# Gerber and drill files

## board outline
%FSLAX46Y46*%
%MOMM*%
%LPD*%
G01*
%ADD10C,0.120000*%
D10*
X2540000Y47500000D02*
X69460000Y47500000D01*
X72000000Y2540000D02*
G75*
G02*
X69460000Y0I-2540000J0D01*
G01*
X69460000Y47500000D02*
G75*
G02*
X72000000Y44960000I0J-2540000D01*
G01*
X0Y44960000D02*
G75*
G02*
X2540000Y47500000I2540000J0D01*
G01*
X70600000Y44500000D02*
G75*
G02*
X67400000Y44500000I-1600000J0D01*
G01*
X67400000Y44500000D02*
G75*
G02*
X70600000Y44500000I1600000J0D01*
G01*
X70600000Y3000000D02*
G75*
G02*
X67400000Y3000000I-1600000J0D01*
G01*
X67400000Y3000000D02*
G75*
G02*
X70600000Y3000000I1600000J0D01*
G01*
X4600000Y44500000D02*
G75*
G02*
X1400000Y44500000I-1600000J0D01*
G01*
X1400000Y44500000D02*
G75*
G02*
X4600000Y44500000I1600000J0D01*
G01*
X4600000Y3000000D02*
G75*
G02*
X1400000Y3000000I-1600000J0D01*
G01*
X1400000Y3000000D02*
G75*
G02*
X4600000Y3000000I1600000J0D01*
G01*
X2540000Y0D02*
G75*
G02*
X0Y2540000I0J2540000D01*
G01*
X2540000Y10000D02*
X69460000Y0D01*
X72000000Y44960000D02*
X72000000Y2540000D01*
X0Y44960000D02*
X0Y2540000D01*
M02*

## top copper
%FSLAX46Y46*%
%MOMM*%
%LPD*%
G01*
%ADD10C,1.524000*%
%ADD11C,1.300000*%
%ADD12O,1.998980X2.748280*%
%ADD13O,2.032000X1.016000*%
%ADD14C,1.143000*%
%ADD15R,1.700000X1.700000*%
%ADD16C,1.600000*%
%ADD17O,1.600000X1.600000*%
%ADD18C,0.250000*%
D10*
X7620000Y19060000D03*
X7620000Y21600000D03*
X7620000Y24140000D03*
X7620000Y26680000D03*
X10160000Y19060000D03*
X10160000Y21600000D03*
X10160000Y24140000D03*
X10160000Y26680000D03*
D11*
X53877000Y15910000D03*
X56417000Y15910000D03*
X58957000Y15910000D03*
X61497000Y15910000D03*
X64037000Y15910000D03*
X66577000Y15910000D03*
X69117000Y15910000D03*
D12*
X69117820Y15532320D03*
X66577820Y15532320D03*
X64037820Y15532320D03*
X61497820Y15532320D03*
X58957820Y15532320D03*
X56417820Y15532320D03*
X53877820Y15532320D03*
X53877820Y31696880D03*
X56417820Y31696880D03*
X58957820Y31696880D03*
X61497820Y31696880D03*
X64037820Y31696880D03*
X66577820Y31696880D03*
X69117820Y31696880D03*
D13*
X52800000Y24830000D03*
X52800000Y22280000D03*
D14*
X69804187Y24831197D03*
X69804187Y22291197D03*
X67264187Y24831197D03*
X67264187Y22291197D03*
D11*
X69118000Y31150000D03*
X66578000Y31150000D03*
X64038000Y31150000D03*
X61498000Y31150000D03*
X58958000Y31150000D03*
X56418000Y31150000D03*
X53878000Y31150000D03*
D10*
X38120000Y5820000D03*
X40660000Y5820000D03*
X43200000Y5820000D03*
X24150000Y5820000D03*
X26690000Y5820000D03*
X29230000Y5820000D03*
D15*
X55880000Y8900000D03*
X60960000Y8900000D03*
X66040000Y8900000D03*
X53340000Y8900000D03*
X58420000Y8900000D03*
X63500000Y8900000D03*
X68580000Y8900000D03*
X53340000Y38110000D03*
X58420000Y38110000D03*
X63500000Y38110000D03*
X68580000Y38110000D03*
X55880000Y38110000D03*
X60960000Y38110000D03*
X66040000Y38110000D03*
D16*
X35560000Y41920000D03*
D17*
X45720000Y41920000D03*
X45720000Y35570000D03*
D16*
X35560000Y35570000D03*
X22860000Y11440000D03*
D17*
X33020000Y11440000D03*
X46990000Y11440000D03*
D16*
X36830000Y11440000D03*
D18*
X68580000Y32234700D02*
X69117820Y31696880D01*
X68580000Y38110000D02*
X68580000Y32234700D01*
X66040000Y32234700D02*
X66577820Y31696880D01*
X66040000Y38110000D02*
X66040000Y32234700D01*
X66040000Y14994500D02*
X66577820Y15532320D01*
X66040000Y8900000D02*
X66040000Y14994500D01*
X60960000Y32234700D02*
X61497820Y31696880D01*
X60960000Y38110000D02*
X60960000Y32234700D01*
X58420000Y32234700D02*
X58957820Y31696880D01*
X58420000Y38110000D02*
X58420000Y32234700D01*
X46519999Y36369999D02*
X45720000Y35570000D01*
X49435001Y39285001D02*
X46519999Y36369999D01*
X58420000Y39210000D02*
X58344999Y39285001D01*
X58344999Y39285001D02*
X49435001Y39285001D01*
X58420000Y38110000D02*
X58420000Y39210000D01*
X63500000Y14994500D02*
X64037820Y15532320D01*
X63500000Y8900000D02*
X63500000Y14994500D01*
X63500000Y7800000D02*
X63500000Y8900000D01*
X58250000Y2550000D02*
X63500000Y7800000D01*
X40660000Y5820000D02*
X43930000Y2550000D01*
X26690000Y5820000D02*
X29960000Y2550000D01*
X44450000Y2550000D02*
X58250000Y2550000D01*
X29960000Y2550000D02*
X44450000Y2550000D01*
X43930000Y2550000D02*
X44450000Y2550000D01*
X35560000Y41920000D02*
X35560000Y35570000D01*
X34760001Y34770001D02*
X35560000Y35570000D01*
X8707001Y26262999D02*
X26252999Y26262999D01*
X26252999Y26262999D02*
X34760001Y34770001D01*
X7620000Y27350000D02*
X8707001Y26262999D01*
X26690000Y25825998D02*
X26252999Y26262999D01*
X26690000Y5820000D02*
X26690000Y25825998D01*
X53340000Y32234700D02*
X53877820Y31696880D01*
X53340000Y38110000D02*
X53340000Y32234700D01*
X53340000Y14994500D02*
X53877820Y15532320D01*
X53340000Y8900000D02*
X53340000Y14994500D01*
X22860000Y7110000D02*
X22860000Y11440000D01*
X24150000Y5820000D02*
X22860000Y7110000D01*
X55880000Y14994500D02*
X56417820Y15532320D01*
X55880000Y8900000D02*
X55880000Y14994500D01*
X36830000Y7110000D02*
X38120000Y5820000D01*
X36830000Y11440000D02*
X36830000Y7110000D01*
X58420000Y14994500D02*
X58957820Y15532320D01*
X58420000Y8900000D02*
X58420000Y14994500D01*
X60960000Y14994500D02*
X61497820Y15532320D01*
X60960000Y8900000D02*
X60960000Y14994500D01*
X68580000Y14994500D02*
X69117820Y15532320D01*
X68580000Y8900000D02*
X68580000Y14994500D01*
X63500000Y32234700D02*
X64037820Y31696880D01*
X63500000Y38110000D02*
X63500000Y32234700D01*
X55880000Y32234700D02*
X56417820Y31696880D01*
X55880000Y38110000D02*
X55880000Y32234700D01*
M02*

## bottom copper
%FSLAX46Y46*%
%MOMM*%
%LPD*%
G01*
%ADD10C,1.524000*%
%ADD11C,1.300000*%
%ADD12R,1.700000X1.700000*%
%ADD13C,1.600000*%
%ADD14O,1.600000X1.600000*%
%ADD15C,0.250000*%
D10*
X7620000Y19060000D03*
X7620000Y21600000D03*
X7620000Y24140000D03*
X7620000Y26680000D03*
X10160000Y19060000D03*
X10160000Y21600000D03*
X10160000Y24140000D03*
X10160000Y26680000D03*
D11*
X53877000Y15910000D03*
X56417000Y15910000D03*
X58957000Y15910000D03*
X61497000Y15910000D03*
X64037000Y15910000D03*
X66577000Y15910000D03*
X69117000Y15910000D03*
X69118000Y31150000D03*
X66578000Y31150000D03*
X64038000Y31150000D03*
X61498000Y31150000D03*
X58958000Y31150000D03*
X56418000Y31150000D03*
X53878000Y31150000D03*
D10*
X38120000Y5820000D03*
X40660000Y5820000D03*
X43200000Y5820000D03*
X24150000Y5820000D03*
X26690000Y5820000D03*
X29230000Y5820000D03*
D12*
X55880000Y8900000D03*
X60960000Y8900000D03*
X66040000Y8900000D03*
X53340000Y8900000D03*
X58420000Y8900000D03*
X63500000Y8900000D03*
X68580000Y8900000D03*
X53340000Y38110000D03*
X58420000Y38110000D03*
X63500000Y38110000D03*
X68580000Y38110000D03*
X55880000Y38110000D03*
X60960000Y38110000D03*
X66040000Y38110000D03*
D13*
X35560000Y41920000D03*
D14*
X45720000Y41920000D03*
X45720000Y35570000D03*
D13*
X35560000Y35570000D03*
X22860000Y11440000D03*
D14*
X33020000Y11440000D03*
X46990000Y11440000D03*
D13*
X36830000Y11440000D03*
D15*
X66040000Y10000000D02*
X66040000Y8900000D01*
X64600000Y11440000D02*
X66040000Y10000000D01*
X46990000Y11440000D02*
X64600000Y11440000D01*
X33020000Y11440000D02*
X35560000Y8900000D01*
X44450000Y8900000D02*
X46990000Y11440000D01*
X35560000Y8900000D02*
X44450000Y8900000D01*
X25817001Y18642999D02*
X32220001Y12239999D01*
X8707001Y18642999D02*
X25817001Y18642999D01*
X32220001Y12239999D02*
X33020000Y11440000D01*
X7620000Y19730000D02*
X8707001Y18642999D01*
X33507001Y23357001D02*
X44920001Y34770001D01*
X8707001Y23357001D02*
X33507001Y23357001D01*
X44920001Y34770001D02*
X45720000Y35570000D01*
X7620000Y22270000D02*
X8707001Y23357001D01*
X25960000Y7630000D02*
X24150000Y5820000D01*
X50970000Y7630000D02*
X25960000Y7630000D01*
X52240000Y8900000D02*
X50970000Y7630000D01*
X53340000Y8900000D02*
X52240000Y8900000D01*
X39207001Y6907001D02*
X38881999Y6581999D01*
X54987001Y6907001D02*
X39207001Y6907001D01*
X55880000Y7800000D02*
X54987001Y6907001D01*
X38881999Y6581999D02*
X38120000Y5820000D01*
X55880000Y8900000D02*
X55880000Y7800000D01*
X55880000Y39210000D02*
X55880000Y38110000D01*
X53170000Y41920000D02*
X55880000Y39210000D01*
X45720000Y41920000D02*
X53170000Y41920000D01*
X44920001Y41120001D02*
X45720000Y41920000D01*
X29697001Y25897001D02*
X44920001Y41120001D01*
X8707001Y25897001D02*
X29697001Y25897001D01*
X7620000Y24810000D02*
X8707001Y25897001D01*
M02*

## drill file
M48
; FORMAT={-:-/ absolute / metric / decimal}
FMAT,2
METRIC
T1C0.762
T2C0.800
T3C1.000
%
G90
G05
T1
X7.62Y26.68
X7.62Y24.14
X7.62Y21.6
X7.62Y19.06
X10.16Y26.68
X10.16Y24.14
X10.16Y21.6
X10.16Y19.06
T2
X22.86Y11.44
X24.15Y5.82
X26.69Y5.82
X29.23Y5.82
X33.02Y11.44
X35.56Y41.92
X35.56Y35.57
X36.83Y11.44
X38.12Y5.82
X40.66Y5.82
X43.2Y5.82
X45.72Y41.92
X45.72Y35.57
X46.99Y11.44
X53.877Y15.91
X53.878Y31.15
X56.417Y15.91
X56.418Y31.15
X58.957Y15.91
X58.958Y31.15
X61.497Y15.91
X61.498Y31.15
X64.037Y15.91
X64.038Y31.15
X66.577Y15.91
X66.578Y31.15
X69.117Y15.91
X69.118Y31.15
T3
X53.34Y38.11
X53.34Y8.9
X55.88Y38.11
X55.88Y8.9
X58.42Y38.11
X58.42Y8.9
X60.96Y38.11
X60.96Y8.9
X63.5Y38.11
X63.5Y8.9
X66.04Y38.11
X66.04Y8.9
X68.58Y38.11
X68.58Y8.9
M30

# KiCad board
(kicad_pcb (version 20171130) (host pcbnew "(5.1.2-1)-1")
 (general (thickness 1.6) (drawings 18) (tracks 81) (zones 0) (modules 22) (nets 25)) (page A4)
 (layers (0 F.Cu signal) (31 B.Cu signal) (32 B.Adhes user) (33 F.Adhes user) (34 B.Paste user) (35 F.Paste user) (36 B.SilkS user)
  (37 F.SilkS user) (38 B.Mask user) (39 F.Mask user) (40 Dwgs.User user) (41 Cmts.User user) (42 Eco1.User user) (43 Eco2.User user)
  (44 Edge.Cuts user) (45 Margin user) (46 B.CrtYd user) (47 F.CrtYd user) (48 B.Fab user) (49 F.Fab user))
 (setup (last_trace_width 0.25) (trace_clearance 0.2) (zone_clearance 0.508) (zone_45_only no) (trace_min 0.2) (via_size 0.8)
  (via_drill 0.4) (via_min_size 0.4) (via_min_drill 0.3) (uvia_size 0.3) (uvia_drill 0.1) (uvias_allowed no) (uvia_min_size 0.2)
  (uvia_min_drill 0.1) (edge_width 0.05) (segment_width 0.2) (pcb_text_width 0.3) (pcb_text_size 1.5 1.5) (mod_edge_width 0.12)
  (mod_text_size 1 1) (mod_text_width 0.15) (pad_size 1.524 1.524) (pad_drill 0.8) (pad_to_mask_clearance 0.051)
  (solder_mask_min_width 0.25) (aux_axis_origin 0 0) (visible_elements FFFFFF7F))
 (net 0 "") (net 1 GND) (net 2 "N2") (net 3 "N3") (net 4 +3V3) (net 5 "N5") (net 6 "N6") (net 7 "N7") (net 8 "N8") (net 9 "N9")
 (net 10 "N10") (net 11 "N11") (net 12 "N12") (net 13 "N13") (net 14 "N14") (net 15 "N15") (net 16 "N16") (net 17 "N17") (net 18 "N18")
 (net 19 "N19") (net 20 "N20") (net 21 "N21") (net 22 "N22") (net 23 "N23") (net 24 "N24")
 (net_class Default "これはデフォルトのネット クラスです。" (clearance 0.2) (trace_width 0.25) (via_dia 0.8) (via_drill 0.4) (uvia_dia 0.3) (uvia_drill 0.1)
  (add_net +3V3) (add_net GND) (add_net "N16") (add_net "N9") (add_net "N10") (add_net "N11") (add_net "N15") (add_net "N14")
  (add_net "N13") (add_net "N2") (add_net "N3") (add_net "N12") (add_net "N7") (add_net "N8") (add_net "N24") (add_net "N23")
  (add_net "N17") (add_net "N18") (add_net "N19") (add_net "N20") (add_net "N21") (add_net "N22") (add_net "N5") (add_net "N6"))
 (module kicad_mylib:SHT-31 (layer F.Cu) (at 6.35 -17.79)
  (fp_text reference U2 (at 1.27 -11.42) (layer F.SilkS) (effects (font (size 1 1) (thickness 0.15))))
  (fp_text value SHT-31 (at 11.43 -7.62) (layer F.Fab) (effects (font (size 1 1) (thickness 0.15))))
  (pad 1 thru_hole circle (at 1.27 -1.27) (size 1.524 1.524) (drill 0.762) (layers *.Cu *.Mask) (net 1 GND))
  (pad 2 thru_hole circle (at 1.27 -3.81) (size 1.524 1.524) (drill 0.762) (layers *.Cu *.Mask) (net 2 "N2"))
  (pad 3 thru_hole circle (at 1.27 -6.35) (size 1.524 1.524) (drill 0.762) (layers *.Cu *.Mask) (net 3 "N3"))
  (pad 4 thru_hole circle (at 1.27 -8.89) (size 1.524 1.524) (drill 0.762) (layers *.Cu *.Mask) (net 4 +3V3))
  (pad 5 thru_hole circle (at 3.81 -1.27) (size 1.524 1.524) (drill 0.762) (layers *.Cu *.Mask) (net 1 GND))
  (pad 6 thru_hole circle (at 3.81 -3.81) (size 1.524 1.524) (drill 0.762) (layers *.Cu *.Mask) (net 1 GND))
  (pad 7 thru_hole circle (at 3.81 -6.35) (size 1.524 1.524) (drill 0.762) (layers *.Cu *.Mask) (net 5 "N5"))
  (pad 8 thru_hole circle (at 3.81 -8.89) (size 1.524 1.524) (drill 0.762) (layers *.Cu *.Mask) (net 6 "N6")))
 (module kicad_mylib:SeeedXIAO (layer F.Cu) (at 51 -32.53 270)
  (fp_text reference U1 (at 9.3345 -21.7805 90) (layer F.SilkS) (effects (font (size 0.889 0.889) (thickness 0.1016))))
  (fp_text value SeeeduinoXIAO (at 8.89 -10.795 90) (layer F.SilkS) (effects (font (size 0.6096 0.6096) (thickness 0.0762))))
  (pad 8 thru_hole circle (at 16.62 -2.877 270) (size 1.3 1.3) (drill 0.8) (layers *.Cu *.Mask) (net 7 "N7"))
  (pad 9 thru_hole circle (at 16.62 -5.417 270) (size 1.3 1.3) (drill 0.8) (layers *.Cu *.Mask) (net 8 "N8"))
  (pad 10 thru_hole circle (at 16.62 -7.957 270) (size 1.3 1.3) (drill 0.8) (layers *.Cu *.Mask) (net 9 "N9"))
  (pad 11 thru_hole circle (at 16.62 -10.497 270) (size 1.3 1.3) (drill 0.8) (layers *.Cu *.Mask) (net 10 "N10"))
  (pad 12 thru_hole circle (at 16.62 -13.037 270) (size 1.3 1.3) (drill 0.8) (layers *.Cu *.Mask) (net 4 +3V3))
  (pad 13 thru_hole circle (at 16.62 -15.577 270) (size 1.3 1.3) (drill 0.8) (layers *.Cu *.Mask) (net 1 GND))
  (pad 14 thru_hole circle (at 16.62 -18.117 270) (size 1.3 1.3) (drill 0.8) (layers *.Cu *.Mask) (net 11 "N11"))
  (pad 14 smd oval (at 16.99768 -18.11782 270) (size 2.74828 1.99898) (layers F.Cu F.Paste F.Mask) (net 11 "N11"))
  (pad 13 smd oval (at 16.99768 -15.57782 270) (size 2.74828 1.99898) (layers F.Cu F.Paste F.Mask) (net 1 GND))
  (pad 12 smd oval (at 16.99768 -13.03782 270) (size 2.74828 1.99898) (layers F.Cu F.Paste F.Mask) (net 4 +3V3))
  (pad 11 smd oval (at 16.99768 -10.49782 270) (size 2.74828 1.99898) (layers F.Cu F.Paste F.Mask) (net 10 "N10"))
  (pad 10 smd oval (at 16.99768 -7.95782 270) (size 2.74828 1.99898) (layers F.Cu F.Paste F.Mask) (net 9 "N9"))
  (pad 9 smd oval (at 16.99768 -5.41782 270) (size 2.74828 1.99898) (layers F.Cu F.Paste F.Mask) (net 8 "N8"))
  (pad 8 smd oval (at 16.99768 -2.87782 270) (size 2.74828 1.99898) (layers F.Cu F.Paste F.Mask) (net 7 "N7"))
  (pad 7 smd oval (at 0.83312 -2.87782 270) (size 2.74828 1.99898) (layers F.Cu F.Paste F.Mask) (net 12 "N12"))
  (pad 6 smd oval (at 0.83312 -5.41782 270) (size 2.74828 1.99898) (layers F.Cu F.Paste F.Mask) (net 3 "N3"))
  (pad 5 smd oval (at 0.83312 -7.95782 270) (size 2.74828 1.99898) (layers F.Cu F.Paste F.Mask) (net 2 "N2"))
  (pad 4 smd oval (at 0.83312 -10.49782 270) (size 2.74828 1.99898) (layers F.Cu F.Paste F.Mask) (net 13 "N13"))
  (pad 3 smd oval (at 0.83312 -13.03782 270) (size 2.74828 1.99898) (layers F.Cu F.Paste F.Mask) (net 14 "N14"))
  (pad 2 smd oval (at 0.83312 -15.57782 270) (size 2.74828 1.99898) (layers F.Cu F.Paste F.Mask) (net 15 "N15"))
  (pad 1 smd oval (at 0.83312 -18.11782 270) (size 2.74828 1.99898) (layers F.Cu F.Paste F.Mask) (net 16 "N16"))
  (pad 15 smd oval (at 7.7 -1.8) (size 2.032 1.016) (layers F.Cu F.Paste F.Mask) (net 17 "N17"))
  (pad 16 smd oval (at 10.25 -1.8) (size 2.032 1.016) (layers F.Cu F.Paste F.Mask) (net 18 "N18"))
  (pad 17 smd circle (at 7.698803 -18.804187) (size 1.143 1.143) (layers F.Cu F.Paste F.Mask) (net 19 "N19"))
  (pad 18 smd circle (at 10.238803 -18.804187) (size 1.143 1.143) (layers F.Cu F.Paste F.Mask) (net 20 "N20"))
  (pad 19 smd circle (at 7.698803 -16.264187) (size 1.143 1.143) (layers F.Cu F.Paste F.Mask) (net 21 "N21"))
  (pad 20 smd circle (at 10.238803 -16.264187) (size 1.143 1.143) (layers F.Cu F.Paste F.Mask) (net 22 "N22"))
  (pad 1 thru_hole circle (at 1.38 -18.118 270) (size 1.3 1.3) (drill 0.8) (layers *.Cu *.Mask) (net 16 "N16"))
  (pad 2 thru_hole circle (at 1.38 -15.578 270) (size 1.3 1.3) (drill 0.8) (layers *.Cu *.Mask) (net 15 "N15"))
  (pad 3 thru_hole circle (at 1.38 -13.038 270) (size 1.3 1.3) (drill 0.8) (layers *.Cu *.Mask) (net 14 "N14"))
  (pad 4 thru_hole circle (at 1.38 -10.498 270) (size 1.3 1.3) (drill 0.8) (layers *.Cu *.Mask) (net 13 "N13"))
  (pad 5 thru_hole circle (at 1.38 -7.958 270) (size 1.3 1.3) (drill 0.8) (layers *.Cu *.Mask) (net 2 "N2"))
  (pad 6 thru_hole circle (at 1.38 -5.418 270) (size 1.3 1.3) (drill 0.8) (layers *.Cu *.Mask) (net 3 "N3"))
  (pad 7 thru_hole circle (at 1.38 -2.878 270) (size 1.3 1.3) (drill 0.8) (layers *.Cu *.Mask) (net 12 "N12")))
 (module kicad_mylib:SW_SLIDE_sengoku (layer F.Cu) (at 35.56 -3.82)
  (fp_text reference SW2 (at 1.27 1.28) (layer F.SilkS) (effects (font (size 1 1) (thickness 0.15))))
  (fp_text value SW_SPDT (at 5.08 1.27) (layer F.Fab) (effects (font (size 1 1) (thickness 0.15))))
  (pad 1 thru_hole circle (at 2.56 -2) (size 1.524 1.524) (drill 0.8) (layers *.Cu *.Mask) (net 8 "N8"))
  (pad 2 thru_hole circle (at 5.1 -2) (size 1.524 1.524) (drill 0.8) (layers *.Cu *.Mask) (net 4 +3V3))
  (pad 3 thru_hole circle (at 7.64 -2) (size 1.524 1.524) (drill 0.8) (layers *.Cu *.Mask) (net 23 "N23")))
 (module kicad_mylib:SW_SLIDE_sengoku (layer F.Cu) (at 21.59 -3.82)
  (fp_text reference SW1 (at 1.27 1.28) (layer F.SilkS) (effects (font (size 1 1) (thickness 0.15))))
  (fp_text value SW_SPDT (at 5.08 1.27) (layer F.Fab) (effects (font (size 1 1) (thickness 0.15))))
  (pad 1 thru_hole circle (at 2.56 -2) (size 1.524 1.524) (drill 0.8) (layers *.Cu *.Mask) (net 7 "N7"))
  (pad 2 thru_hole circle (at 5.1 -2) (size 1.524 1.524) (drill 0.8) (layers *.Cu *.Mask) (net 4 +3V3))
  (pad 3 thru_hole circle (at 7.64 -2) (size 1.524 1.524) (drill 0.8) (layers *.Cu *.Mask) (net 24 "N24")))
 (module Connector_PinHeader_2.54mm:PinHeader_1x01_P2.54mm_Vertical (layer F.Cu) (at 55.88 -8.9)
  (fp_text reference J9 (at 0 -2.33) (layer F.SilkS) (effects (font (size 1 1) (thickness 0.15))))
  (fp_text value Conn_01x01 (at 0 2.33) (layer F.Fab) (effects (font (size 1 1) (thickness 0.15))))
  (pad 1 thru_hole rect (at 0 0) (size 1.7 1.7) (drill 1) (layers *.Cu *.Mask) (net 8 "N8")))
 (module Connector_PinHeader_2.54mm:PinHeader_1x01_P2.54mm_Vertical (layer F.Cu) (at 60.96 -8.9)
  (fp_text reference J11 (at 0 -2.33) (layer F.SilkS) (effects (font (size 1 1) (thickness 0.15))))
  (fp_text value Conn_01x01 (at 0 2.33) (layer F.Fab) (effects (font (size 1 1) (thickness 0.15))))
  (pad 1 thru_hole rect (at 0 0) (size 1.7 1.7) (drill 1) (layers *.Cu *.Mask) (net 10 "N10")))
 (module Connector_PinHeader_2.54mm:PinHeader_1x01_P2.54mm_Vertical (layer F.Cu) (at 66.04 -8.9)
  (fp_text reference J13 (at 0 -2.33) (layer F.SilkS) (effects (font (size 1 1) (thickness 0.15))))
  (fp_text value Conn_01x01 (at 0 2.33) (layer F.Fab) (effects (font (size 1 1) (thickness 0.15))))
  (pad 1 thru_hole rect (at 0 0) (size 1.7 1.7) (drill 1) (layers *.Cu *.Mask) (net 1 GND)))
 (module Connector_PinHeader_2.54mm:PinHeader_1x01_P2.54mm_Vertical (layer F.Cu) (at 53.34 -8.9)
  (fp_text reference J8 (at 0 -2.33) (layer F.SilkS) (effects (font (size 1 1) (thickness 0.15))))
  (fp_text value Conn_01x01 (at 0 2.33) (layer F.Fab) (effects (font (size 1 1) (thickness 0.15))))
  (pad 1 thru_hole rect (at 0 0) (size 1.7 1.7) (drill 1) (layers *.Cu *.Mask) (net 7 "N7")))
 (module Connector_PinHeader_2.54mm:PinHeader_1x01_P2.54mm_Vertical (layer F.Cu) (at 58.42 -8.9)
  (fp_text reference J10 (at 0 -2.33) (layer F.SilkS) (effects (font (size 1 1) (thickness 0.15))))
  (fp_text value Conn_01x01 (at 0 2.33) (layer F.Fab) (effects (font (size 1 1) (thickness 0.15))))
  (pad 1 thru_hole rect (at 0 0) (size 1.7 1.7) (drill 1) (layers *.Cu *.Mask) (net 9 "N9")))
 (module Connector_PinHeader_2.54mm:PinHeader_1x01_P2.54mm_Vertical (layer F.Cu) (at 63.5 -8.9)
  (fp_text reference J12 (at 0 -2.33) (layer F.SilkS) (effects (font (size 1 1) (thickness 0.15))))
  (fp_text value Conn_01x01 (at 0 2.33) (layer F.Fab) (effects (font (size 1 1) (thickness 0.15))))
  (pad 1 thru_hole rect (at 0 0) (size 1.7 1.7) (drill 1) (layers *.Cu *.Mask) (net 4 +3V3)))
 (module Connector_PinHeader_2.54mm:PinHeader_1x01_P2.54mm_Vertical (layer F.Cu) (at 68.58 -8.9)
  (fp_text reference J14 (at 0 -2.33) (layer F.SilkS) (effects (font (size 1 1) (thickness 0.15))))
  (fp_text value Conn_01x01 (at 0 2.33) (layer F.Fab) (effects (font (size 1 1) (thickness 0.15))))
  (pad 1 thru_hole rect (at 0 0) (size 1.7 1.7) (drill 1) (layers *.Cu *.Mask) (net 11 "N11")))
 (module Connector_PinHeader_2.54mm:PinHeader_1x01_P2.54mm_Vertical (layer F.Cu) (at 53.34 -38.11)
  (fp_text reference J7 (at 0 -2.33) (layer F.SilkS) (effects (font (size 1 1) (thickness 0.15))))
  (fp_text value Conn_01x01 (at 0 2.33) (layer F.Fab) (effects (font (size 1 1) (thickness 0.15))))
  (pad 1 thru_hole rect (at 0 0) (size 1.7 1.7) (drill 1) (layers *.Cu *.Mask) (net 12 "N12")))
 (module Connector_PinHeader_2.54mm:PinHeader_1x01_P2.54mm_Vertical (layer F.Cu) (at 58.42 -38.11)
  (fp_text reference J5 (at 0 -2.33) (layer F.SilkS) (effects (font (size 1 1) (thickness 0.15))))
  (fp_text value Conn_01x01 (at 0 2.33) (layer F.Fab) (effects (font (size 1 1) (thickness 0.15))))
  (pad 1 thru_hole rect (at 0 0) (size 1.7 1.7) (drill 1) (layers *.Cu *.Mask) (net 2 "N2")))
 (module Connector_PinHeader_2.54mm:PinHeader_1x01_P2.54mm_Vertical (layer F.Cu) (at 63.5 -38.11)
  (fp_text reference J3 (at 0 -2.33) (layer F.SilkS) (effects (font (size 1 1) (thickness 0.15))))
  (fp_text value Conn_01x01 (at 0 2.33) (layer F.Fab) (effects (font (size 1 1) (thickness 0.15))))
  (pad 1 thru_hole rect (at 0 0) (size 1.7 1.7) (drill 1) (layers *.Cu *.Mask) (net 14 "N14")))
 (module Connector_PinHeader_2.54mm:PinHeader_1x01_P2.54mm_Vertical (layer F.Cu) (at 68.58 -38.11)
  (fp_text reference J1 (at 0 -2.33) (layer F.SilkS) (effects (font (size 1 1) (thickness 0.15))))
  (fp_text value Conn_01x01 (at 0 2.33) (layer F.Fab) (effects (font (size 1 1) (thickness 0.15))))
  (pad 1 thru_hole rect (at 0 0) (size 1.7 1.7) (drill 1) (layers *.Cu *.Mask) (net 16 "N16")))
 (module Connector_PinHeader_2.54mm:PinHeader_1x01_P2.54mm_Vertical (layer F.Cu) (at 55.88 -38.11)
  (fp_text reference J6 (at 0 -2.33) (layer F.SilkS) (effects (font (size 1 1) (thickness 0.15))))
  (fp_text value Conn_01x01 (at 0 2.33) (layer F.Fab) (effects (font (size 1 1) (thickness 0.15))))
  (pad 1 thru_hole rect (at 0 0) (size 1.7 1.7) (drill 1) (layers *.Cu *.Mask) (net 3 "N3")))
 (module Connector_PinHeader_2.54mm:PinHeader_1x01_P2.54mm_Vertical (layer F.Cu) (at 60.96 -38.11)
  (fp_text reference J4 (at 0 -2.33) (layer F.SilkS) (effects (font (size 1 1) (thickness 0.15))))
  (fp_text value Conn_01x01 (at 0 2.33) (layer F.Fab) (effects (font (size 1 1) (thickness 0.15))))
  (pad 1 thru_hole rect (at 0 0) (size 1.7 1.7) (drill 1) (layers *.Cu *.Mask) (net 13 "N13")))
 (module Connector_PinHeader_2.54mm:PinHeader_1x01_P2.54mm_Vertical (layer F.Cu) (at 66.04 -38.11)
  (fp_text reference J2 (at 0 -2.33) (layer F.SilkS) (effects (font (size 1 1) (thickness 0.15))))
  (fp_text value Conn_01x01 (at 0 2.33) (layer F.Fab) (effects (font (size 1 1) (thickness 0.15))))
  (pad 1 thru_hole rect (at 0 0) (size 1.7 1.7) (drill 1) (layers *.Cu *.Mask) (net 15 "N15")))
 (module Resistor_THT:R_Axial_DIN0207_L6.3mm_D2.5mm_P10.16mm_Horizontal (layer F.Cu) (at 35.56 -41.92)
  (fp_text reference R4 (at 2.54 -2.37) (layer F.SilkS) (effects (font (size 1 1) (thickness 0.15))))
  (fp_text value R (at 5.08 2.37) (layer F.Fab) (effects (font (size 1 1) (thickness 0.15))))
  (pad 1 thru_hole circle (at 0 0) (size 1.6 1.6) (drill 0.8) (layers *.Cu *.Mask) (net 4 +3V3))
  (pad 2 thru_hole oval (at 10.16 0) (size 1.6 1.6) (drill 0.8) (layers *.Cu *.Mask) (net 3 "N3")))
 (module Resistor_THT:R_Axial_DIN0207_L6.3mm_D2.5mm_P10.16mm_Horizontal (layer F.Cu) (at 35.56 -35.57)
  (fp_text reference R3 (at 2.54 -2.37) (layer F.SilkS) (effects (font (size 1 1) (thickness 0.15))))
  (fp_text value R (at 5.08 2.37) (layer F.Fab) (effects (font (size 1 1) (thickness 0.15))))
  (pad 2 thru_hole oval (at 10.16 0) (size 1.6 1.6) (drill 0.8) (layers *.Cu *.Mask) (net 2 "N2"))
  (pad 1 thru_hole circle (at 0 0) (size 1.6 1.6) (drill 0.8) (layers *.Cu *.Mask) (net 4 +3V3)))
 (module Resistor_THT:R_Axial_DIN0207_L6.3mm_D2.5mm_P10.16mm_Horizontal (layer F.Cu) (at 22.86 -11.44)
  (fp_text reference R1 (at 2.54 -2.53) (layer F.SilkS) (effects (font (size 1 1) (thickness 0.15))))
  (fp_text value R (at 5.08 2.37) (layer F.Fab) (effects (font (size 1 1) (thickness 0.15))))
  (pad 1 thru_hole circle (at 0 0) (size 1.6 1.6) (drill 0.8) (layers *.Cu *.Mask) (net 7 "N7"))
  (pad 2 thru_hole oval (at 10.16 0) (size 1.6 1.6) (drill 0.8) (layers *.Cu *.Mask) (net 1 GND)))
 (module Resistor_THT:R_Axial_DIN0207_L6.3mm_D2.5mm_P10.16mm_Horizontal (layer F.Cu) (at 36.83 -11.44)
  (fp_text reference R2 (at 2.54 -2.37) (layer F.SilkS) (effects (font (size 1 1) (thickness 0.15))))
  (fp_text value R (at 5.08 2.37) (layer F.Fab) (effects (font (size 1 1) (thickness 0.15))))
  (pad 2 thru_hole oval (at 10.16 0) (size 1.6 1.6) (drill 0.8) (layers *.Cu *.Mask) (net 1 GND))
  (pad 1 thru_hole circle (at 0 0) (size 1.6 1.6) (drill 0.8) (layers *.Cu *.Mask) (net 8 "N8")))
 (gr_line (start 2.54 -47.5) (end 69.46 -47.5) (layer Edge.Cuts) (width 0.12))
 (gr_arc (start 69.46 -2.54) (end 72 -2.54) (angle 90) (layer Edge.Cuts) (width 0.12))
 (gr_arc (start 69.46 -44.96) (end 69.46 -47.5) (angle 90) (layer Edge.Cuts) (width 0.12))
 (gr_arc (start 2.54 -44.96) (end 0 -44.96) (angle 90) (layer Edge.Cuts) (width 0.12))
 (gr_circle (center 69 -44.5) (end 70.6 -44.5) (layer Edge.Cuts) (width 0.12))
 (gr_circle (center 69 -3) (end 70.6 -3) (layer Edge.Cuts) (width 0.12))
 (gr_circle (center 3 -44.5) (end 4.6 -44.5) (layer Edge.Cuts) (width 0.12))
 (gr_circle (center 3 -3) (end 4.6 -3) (layer Edge.Cuts) (width 0.12))
 (gr_arc (start 2.54 -2.54) (end 2.54 0) (angle 90) (layer Edge.Cuts) (width 0.12))
 (gr_line (start 2.54 -0.01) (end 69.46 0) (layer Edge.Cuts) (width 0.12))
 (gr_line (start 72 -44.96) (end 72 -2.54) (layer Edge.Cuts) (width 0.12))
 (gr_line (start 0 -44.96) (end 0 -2.54) (layer Edge.Cuts) (width 0.12))
 (segment (start 68.58 -32.2347) (end 69.11782 -31.69688) (width 0.25) (layer F.Cu) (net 16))
 (segment (start 68.58 -38.11) (end 68.58 -32.2347) (width 0.25) (layer F.Cu) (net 16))
 (segment (start 66.04 -32.2347) (end 66.57782 -31.69688) (width 0.25) (layer F.Cu) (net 15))
 (segment (start 66.04 -38.11) (end 66.04 -32.2347) (width 0.25) (layer F.Cu) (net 15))
 (segment (start 66.04 -14.9945) (end 66.57782 -15.53232) (width 0.25) (layer F.Cu) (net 1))
 (segment (start 66.04 -8.9) (end 66.04 -14.9945) (width 0.25) (layer F.Cu) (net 1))
 (segment (start 66.04 -10) (end 66.04 -8.9) (width 0.25) (layer B.Cu) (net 1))
 (segment (start 64.6 -11.44) (end 66.04 -10) (width 0.25) (layer B.Cu) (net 1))
 (segment (start 46.99 -11.44) (end 64.6 -11.44) (width 0.25) (layer B.Cu) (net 1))
 (segment (start 33.02 -11.44) (end 35.56 -8.9) (width 0.25) (layer B.Cu) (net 1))
 (segment (start 44.45 -8.9) (end 46.99 -11.44) (width 0.25) (layer B.Cu) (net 1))
 (segment (start 35.56 -8.9) (end 44.45 -8.9) (width 0.25) (layer B.Cu) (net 1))
 (segment (start 25.817001 -18.642999) (end 32.220001 -12.239999) (width 0.25) (layer B.Cu) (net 1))
 (segment (start 8.707001 -18.642999) (end 25.817001 -18.642999) (width 0.25) (layer B.Cu) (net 1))
 (segment (start 32.220001 -12.239999) (end 33.02 -11.44) (width 0.25) (layer B.Cu) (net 1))
 (segment (start 7.62 -19.73) (end 8.707001 -18.642999) (width 0.25) (layer B.Cu) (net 1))
 (segment (start 60.96 -32.2347) (end 61.49782 -31.69688) (width 0.25) (layer F.Cu) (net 13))
 (segment (start 60.96 -38.11) (end 60.96 -32.2347) (width 0.25) (layer F.Cu) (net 13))
 (segment (start 58.42 -32.2347) (end 58.95782 -31.69688) (width 0.25) (layer F.Cu) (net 2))
 (segment (start 58.42 -38.11) (end 58.42 -32.2347) (width 0.25) (layer F.Cu) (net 2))
 (segment (start 46.519999 -36.369999) (end 45.72 -35.57) (width 0.25) (layer F.Cu) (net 2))
 (segment (start 49.435001 -39.285001) (end 46.519999 -36.369999) (width 0.25) (layer F.Cu) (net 2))
 (segment (start 58.42 -39.21) (end 58.344999 -39.285001) (width 0.25) (layer F.Cu) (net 2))
 (segment (start 58.344999 -39.285001) (end 49.435001 -39.285001) (width 0.25) (layer F.Cu) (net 2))
 (segment (start 58.42 -38.11) (end 58.42 -39.21) (width 0.25) (layer F.Cu) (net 2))
 (segment (start 33.507001 -23.357001) (end 44.920001 -34.770001) (width 0.25) (layer B.Cu) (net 2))
 (segment (start 8.707001 -23.357001) (end 33.507001 -23.357001) (width 0.25) (layer B.Cu) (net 2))
 (segment (start 44.920001 -34.770001) (end 45.72 -35.57) (width 0.25) (layer B.Cu) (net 2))
 (segment (start 7.62 -22.27) (end 8.707001 -23.357001) (width 0.25) (layer B.Cu) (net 2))
 (segment (start 63.5 -14.9945) (end 64.03782 -15.53232) (width 0.25) (layer F.Cu) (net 4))
 (segment (start 63.5 -8.9) (end 63.5 -14.9945) (width 0.25) (layer F.Cu) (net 4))
 (segment (start 63.5 -7.8) (end 63.5 -8.9) (width 0.25) (layer F.Cu) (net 4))
 (segment (start 58.25 -2.55) (end 63.5 -7.8) (width 0.25) (layer F.Cu) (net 4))
 (segment (start 40.66 -5.82) (end 43.93 -2.55) (width 0.25) (layer F.Cu) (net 4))
 (segment (start 26.69 -5.82) (end 29.96 -2.55) (width 0.25) (layer F.Cu) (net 4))
 (segment (start 44.45 -2.55) (end 58.25 -2.55) (width 0.25) (layer F.Cu) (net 4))
 (segment (start 29.96 -2.55) (end 44.45 -2.55) (width 0.25) (layer F.Cu) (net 4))
 (segment (start 43.93 -2.55) (end 44.45 -2.55) (width 0.25) (layer F.Cu) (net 4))
 (segment (start 35.56 -41.92) (end 35.56 -35.57) (width 0.25) (layer F.Cu) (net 4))
 (segment (start 34.760001 -34.770001) (end 35.56 -35.57) (width 0.25) (layer F.Cu) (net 4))
 (segment (start 8.707001 -26.262999) (end 26.252999 -26.262999) (width 0.25) (layer F.Cu) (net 4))
 (segment (start 26.252999 -26.262999) (end 34.760001 -34.770001) (width 0.25) (layer F.Cu) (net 4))
 (segment (start 7.62 -27.35) (end 8.707001 -26.262999) (width 0.25) (layer F.Cu) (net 4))
 (segment (start 26.69 -25.825998) (end 26.252999 -26.262999) (width 0.25) (layer F.Cu) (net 4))
 (segment (start 26.69 -5.82) (end 26.69 -25.825998) (width 0.25) (layer F.Cu) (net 4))
 (segment (start 53.34 -32.2347) (end 53.87782 -31.69688) (width 0.25) (layer F.Cu) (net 12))
 (segment (start 53.34 -38.11) (end 53.34 -32.2347) (width 0.25) (layer F.Cu) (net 12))
 (segment (start 53.34 -14.9945) (end 53.87782 -15.53232) (width 0.25) (layer F.Cu) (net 7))
 (segment (start 53.34 -8.9) (end 53.34 -14.9945) (width 0.25) (layer F.Cu) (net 7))
 (segment (start 22.86 -7.11) (end 22.86 -11.44) (width 0.25) (layer F.Cu) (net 7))
 (segment (start 24.15 -5.82) (end 22.86 -7.11) (width 0.25) (layer F.Cu) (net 7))
 (segment (start 25.96 -7.63) (end 24.15 -5.82) (width 0.25) (layer B.Cu) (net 7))
 (segment (start 50.97 -7.63) (end 25.96 -7.63) (width 0.25) (layer B.Cu) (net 7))
 (segment (start 52.24 -8.9) (end 50.97 -7.63) (width 0.25) (layer B.Cu) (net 7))
 (segment (start 53.34 -8.9) (end 52.24 -8.9) (width 0.25) (layer B.Cu) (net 7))
 (segment (start 55.88 -14.9945) (end 56.41782 -15.53232) (width 0.25) (layer F.Cu) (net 8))
 (segment (start 55.88 -8.9) (end 55.88 -14.9945) (width 0.25) (layer F.Cu) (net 8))
 (segment (start 36.83 -7.11) (end 38.12 -5.82) (width 0.25) (layer F.Cu) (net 8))
 (segment (start 36.83 -11.44) (end 36.83 -7.11) (width 0.25) (layer F.Cu) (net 8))
 (segment (start 39.207001 -6.907001) (end 38.881999 -6.581999) (width 0.25) (layer B.Cu) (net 8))
 (segment (start 54.987001 -6.907001) (end 39.207001 -6.907001) (width 0.25) (layer B.Cu) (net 8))
 (segment (start 55.88 -7.8) (end 54.987001 -6.907001) (width 0.25) (layer B.Cu) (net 8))
 (segment (start 38.881999 -6.581999) (end 38.12 -5.82) (width 0.25) (layer B.Cu) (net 8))
 (segment (start 55.88 -8.9) (end 55.88 -7.8) (width 0.25) (layer B.Cu) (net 8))
 (segment (start 58.42 -14.9945) (end 58.95782 -15.53232) (width 0.25) (layer F.Cu) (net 9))
 (segment (start 58.42 -8.9) (end 58.42 -14.9945) (width 0.25) (layer F.Cu) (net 9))
 (segment (start 60.96 -14.9945) (end 61.49782 -15.53232) (width 0.25) (layer F.Cu) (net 10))
 (segment (start 60.96 -8.9) (end 60.96 -14.9945) (width 0.25) (layer F.Cu) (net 10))
 (segment (start 68.58 -14.9945) (end 69.11782 -15.53232) (width 0.25) (layer F.Cu) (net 11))
 (segment (start 68.58 -8.9) (end 68.58 -14.9945) (width 0.25) (layer F.Cu) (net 11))
 (segment (start 63.5 -32.2347) (end 64.03782 -31.69688) (width 0.25) (layer F.Cu) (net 14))
 (segment (start 63.5 -38.11) (end 63.5 -32.2347) (width 0.25) (layer F.Cu) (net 14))
 (segment (start 55.88 -32.2347) (end 56.41782 -31.69688) (width 0.25) (layer F.Cu) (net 3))
 (segment (start 55.88 -38.11) (end 55.88 -32.2347) (width 0.25) (layer F.Cu) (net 3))
 (segment (start 55.88 -39.21) (end 55.88 -38.11) (width 0.25) (layer B.Cu) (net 3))
 (segment (start 53.17 -41.92) (end 55.88 -39.21) (width 0.25) (layer B.Cu) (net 3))
 (segment (start 45.72 -41.92) (end 53.17 -41.92) (width 0.25) (layer B.Cu) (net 3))
 (segment (start 44.920001 -41.120001) (end 45.72 -41.92) (width 0.25) (layer B.Cu) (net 3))
 (segment (start 29.697001 -25.897001) (end 44.920001 -41.120001) (width 0.25) (layer B.Cu) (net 3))
 (segment (start 8.707001 -25.897001) (end 29.697001 -25.897001) (width 0.25) (layer B.Cu) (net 3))
 (segment (start 7.62 -24.81) (end 8.707001 -25.897001) (width 0.25) (layer B.Cu) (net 3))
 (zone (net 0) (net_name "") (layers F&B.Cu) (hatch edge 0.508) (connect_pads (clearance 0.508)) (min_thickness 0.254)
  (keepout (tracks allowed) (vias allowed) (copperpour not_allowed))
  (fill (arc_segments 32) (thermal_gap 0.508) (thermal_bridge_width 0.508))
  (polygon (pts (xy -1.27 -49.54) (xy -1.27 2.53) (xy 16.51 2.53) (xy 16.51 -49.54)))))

